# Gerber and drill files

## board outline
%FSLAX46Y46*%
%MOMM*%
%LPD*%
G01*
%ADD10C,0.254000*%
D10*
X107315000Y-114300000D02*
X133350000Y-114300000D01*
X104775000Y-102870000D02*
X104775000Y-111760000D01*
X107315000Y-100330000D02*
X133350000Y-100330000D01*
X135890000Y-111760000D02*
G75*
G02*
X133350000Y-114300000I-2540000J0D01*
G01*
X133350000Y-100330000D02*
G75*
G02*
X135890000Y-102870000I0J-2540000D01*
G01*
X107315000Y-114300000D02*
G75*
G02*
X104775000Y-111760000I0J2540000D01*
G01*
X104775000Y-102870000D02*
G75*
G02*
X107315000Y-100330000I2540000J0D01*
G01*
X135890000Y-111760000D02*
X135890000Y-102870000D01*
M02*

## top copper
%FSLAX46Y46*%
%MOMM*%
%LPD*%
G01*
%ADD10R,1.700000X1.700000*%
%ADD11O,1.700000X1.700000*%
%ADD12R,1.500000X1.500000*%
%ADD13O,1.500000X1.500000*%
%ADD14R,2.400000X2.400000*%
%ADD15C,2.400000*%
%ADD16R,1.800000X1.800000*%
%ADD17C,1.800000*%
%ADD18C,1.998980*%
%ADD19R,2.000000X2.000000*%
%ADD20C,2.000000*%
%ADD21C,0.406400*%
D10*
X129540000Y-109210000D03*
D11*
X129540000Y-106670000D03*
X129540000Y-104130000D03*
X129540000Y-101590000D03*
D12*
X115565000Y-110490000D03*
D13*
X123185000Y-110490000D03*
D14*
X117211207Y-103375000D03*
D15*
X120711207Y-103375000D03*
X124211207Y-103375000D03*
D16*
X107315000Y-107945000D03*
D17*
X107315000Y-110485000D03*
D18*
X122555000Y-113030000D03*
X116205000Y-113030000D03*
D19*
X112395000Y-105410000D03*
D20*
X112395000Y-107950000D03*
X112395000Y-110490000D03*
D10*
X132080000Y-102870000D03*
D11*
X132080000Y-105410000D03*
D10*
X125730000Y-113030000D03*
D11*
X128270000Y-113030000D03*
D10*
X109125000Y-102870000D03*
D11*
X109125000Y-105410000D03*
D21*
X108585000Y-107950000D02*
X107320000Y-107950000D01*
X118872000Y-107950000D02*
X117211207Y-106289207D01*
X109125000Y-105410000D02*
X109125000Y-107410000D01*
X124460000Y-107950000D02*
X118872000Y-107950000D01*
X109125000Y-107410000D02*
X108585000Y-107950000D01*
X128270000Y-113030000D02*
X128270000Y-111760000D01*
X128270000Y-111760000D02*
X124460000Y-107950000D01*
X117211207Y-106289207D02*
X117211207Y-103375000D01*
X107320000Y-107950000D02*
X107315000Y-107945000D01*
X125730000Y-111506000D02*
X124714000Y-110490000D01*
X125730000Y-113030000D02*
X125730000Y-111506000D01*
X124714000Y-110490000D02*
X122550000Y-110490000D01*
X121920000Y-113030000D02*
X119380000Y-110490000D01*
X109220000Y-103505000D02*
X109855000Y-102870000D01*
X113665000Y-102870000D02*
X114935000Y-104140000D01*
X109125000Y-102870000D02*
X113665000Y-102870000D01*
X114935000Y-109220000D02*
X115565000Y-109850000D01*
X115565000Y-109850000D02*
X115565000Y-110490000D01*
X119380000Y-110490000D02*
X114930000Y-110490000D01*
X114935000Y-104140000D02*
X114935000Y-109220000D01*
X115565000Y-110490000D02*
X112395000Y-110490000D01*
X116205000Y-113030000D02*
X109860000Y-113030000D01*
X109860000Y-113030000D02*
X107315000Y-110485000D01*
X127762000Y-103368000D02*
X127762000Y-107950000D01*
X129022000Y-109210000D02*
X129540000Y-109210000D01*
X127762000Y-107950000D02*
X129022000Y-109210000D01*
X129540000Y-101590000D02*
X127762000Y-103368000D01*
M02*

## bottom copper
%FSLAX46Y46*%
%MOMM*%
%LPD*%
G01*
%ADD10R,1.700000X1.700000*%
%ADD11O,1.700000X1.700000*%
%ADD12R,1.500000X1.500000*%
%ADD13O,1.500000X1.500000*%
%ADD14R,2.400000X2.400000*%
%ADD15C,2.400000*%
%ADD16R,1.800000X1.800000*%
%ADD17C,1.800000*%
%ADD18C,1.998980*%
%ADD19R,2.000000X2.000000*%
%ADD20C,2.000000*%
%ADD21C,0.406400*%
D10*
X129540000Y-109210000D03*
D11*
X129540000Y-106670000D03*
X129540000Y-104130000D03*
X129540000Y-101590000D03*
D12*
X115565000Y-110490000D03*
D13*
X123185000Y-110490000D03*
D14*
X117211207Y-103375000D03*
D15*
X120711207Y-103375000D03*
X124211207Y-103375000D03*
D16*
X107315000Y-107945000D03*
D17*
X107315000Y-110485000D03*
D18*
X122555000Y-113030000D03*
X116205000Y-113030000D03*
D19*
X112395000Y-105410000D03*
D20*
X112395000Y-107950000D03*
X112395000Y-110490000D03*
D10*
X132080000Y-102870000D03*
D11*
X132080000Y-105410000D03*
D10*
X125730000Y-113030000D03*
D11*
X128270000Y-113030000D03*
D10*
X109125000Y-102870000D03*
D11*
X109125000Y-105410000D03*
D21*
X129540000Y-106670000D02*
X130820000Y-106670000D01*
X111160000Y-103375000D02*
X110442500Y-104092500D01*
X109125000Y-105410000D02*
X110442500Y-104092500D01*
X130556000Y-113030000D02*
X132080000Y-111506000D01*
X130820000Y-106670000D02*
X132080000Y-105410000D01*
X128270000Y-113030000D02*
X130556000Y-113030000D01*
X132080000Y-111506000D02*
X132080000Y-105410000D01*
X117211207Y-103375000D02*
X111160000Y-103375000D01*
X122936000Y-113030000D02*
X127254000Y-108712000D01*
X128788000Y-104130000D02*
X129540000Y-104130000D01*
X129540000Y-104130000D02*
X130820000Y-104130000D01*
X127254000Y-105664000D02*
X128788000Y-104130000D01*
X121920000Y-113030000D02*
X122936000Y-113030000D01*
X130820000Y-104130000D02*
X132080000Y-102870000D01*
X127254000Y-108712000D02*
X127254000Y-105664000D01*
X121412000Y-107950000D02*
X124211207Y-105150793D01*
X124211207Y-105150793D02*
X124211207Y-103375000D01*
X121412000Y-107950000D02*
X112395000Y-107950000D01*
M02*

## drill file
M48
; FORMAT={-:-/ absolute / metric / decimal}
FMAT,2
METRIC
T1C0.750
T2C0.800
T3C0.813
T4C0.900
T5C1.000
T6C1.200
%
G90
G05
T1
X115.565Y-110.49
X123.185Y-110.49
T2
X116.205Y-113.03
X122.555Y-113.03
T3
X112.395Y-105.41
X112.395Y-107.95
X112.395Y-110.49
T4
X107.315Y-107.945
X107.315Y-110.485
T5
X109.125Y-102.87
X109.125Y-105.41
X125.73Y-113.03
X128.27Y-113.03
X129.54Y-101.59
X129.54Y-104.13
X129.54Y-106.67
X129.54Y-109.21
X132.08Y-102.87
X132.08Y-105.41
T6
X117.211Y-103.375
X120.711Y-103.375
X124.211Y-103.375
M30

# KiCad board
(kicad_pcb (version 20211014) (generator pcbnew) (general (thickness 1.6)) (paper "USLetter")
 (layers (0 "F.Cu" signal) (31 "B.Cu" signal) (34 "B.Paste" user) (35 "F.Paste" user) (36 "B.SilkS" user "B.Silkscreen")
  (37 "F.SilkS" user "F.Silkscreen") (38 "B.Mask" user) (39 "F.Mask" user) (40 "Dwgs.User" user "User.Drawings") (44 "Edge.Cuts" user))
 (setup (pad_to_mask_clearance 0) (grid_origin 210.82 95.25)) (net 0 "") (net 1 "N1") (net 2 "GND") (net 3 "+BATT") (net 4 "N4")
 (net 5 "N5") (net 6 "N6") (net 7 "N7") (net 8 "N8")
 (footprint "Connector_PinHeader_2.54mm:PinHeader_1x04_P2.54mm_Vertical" (layer "F.Cu") (at 129.54 109.21 180)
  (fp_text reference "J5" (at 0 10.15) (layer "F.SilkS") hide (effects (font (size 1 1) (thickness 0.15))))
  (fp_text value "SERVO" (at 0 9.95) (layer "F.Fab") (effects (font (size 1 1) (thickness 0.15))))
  (pad "1" thru_hole rect (at 0 0 180) (size 1.7 1.7) (drill 1) (layers *.Cu *.Mask) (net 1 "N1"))
  (pad "2" thru_hole oval (at 0 2.54 180) (size 1.7 1.7) (drill 1) (layers *.Cu *.Mask) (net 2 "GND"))
  (pad "3" thru_hole oval (at 0 5.08 180) (size 1.7 1.7) (drill 1) (layers *.Cu *.Mask) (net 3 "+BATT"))
  (pad "4" thru_hole oval (at 0 7.62 180) (size 1.7 1.7) (drill 1) (layers *.Cu *.Mask) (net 1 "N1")))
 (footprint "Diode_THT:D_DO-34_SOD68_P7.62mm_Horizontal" (layer "F.Cu") (at 115.565 110.49)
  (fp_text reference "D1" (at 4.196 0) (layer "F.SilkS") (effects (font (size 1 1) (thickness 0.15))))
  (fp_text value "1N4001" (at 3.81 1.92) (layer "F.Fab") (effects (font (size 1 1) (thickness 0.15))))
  (pad "1" thru_hole rect (at 0 0) (size 1.5 1.5) (drill 0.75) (layers *.Cu *.Mask) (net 3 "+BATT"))
  (pad "2" thru_hole oval (at 7.62 0) (size 1.5 1.5) (drill 0.75) (layers *.Cu *.Mask) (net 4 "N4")))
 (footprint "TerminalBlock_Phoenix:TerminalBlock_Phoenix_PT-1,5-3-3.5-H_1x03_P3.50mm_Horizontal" (layer "F.Cu") (at 117.211207 103.375)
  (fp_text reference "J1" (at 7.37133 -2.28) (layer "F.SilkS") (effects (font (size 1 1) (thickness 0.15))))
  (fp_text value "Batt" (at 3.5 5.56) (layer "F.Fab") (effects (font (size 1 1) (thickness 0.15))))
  (pad "1" thru_hole rect (at 0 0) (size 2.4 2.4) (drill 1.2) (layers *.Cu *.Mask) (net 2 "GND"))
  (pad "2" thru_hole circle (at 3.5 0) (size 2.4 2.4) (drill 1.2) (layers *.Cu *.Mask) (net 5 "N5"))
  (pad "3" thru_hole circle (at 7 0) (size 2.4 2.4) (drill 1.2) (layers *.Cu *.Mask) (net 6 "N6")))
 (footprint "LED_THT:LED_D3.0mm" (layer "F.Cu") (at 107.315 107.945 -90)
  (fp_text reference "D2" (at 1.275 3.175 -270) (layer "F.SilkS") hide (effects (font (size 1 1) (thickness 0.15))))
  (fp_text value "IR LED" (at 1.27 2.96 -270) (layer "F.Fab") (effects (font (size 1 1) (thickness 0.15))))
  (pad "1" thru_hole rect (at 0 0 270) (size 1.8 1.8) (drill 0.9) (layers *.Cu *.Mask) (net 2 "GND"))
  (pad "2" thru_hole circle (at 2.54 0 270) (size 1.8 1.8) (drill 0.9) (layers *.Cu *.Mask) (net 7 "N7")))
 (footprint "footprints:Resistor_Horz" (layer "F.Cu") (at 119.38 113.03 180)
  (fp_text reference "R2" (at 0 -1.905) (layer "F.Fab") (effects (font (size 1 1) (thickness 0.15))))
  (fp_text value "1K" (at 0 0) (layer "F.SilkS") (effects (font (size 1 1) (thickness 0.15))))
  (pad "1" thru_hole circle (at -3.175 0 180) (size 1.99898 1.99898) (drill 0.8) (layers *.Cu *.SilkS *.Mask) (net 3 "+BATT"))
  (pad "2" thru_hole circle (at 3.175 0 180) (size 1.99898 1.99898) (drill 0.8) (layers *.Cu *.SilkS *.Mask) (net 7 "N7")))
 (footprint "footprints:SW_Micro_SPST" (layer "F.Cu") (at 112.395 107.95 -90)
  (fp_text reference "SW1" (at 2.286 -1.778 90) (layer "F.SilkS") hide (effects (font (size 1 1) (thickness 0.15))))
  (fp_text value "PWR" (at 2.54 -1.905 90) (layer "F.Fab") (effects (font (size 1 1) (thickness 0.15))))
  (pad "1" thru_hole rect (at -2.54 0 270) (size 2 2) (drill 0.8128) (layers *.Cu *.Mask "F.SilkS") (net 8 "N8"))
  (pad "2" thru_hole circle (at 0 0 270) (size 2 2) (drill 0.8128) (layers *.Cu *.Mask "F.SilkS") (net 6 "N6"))
  (pad "3" thru_hole circle (at 2.54 0 270) (size 2 2) (drill 0.8128) (layers *.Cu *.Mask "F.SilkS") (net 3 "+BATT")))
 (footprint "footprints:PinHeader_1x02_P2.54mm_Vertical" (layer "B.Cu") (at 132.08 102.87 180)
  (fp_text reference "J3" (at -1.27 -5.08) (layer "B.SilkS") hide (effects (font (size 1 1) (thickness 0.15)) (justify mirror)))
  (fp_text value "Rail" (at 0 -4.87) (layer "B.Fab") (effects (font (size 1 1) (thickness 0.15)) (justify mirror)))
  (pad "1" thru_hole rect (at 0 0 180) (size 1.7 1.7) (drill 1) (layers *.Cu *.Mask) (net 3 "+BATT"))
  (pad "2" thru_hole oval (at 0 -2.54 180) (size 1.7 1.7) (drill 1) (layers *.Cu *.Mask) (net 2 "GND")))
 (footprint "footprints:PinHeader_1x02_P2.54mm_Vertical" (layer "B.Cu") (at 125.73 113.03 -90)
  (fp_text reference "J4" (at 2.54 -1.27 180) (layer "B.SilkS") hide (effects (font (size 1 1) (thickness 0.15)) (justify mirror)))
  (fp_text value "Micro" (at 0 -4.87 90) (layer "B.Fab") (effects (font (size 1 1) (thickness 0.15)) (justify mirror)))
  (pad "1" thru_hole rect (at 0 0 270) (size 1.7 1.7) (drill 1) (layers *.Cu *.Mask) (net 4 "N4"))
  (pad "2" thru_hole oval (at 0 -2.54 270) (size 1.7 1.7) (drill 1) (layers *.Cu *.Mask) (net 2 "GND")))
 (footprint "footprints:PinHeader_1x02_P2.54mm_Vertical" (layer "B.Cu") (at 109.125 102.87 180)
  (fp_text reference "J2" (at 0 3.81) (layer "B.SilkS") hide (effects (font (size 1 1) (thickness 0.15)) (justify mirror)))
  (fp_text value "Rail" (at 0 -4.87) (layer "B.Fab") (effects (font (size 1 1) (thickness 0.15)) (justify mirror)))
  (pad "1" thru_hole rect (at 0 0 180) (size 1.7 1.7) (drill 1) (layers *.Cu *.Mask) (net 3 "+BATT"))
  (pad "2" thru_hole oval (at 0 -2.54 180) (size 1.7 1.7) (drill 1) (layers *.Cu *.Mask) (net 2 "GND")))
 (gr_line (start 107.315 114.3) (end 133.35 114.3) (layer "Edge.Cuts") (width 0.254))
 (gr_line (start 104.775 102.87) (end 104.775 111.76) (layer "Edge.Cuts") (width 0.254))
 (gr_line (start 107.315 100.33) (end 133.35 100.33) (layer "Edge.Cuts") (width 0.254))
 (gr_arc (start 135.89 111.76) (mid 135.146051 113.556051) (end 133.35 114.3) (layer "Edge.Cuts") (width 0.254))
 (gr_arc (start 133.35 100.33) (mid 135.146051 101.073949) (end 135.89 102.87) (layer "Edge.Cuts") (width 0.254))
 (gr_arc (start 107.315 114.3) (mid 105.518949 113.556051) (end 104.775 111.76) (layer "Edge.Cuts") (width 0.254))
 (gr_arc (start 104.775 102.87) (mid 105.518949 101.073949) (end 107.315 100.33) (layer "Edge.Cuts") (width 0.254))
 (gr_line (start 135.89 111.76) (end 135.89 102.87) (layer "Edge.Cuts") (width 0.254))
 (segment (start 108.585 107.95) (end 107.32 107.95) (width 0.4064) (layer "F.Cu") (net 2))
 (segment (start 118.872 107.95) (end 117.211207 106.289207) (width 0.4064) (layer "F.Cu") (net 2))
 (segment (start 109.125 105.41) (end 109.125 107.41) (width 0.4064) (layer "F.Cu") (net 2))
 (segment (start 124.46 107.95) (end 118.872 107.95) (width 0.4064) (layer "F.Cu") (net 2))
 (segment (start 109.125 107.41) (end 108.585 107.95) (width 0.4064) (layer "F.Cu") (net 2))
 (segment (start 128.27 113.03) (end 128.27 111.76) (width 0.4064) (layer "F.Cu") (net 2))
 (segment (start 128.27 111.76) (end 124.46 107.95) (width 0.4064) (layer "F.Cu") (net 2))
 (segment (start 117.211207 106.289207) (end 117.211207 103.375) (width 0.4064) (layer "F.Cu") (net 2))
 (segment (start 107.32 107.95) (end 107.315 107.945) (width 0.4064) (layer "F.Cu") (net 2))
 (segment (start 129.54 106.67) (end 130.82 106.67) (width 0.4064) (layer "B.Cu") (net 2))
 (segment (start 111.16 103.375) (end 110.4425 104.0925) (width 0.4064) (layer "B.Cu") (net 2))
 (segment (start 109.125 105.41) (end 110.4425 104.0925) (width 0.4064) (layer "B.Cu") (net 2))
 (segment (start 130.556 113.03) (end 132.08 111.506) (width 0.4064) (layer "B.Cu") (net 2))
 (segment (start 130.82 106.67) (end 132.08 105.41) (width 0.4064) (layer "B.Cu") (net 2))
 (segment (start 128.27 113.03) (end 130.556 113.03) (width 0.4064) (layer "B.Cu") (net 2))
 (segment (start 132.08 111.506) (end 132.08 105.41) (width 0.4064) (layer "B.Cu") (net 2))
 (segment (start 117.211207 103.375) (end 111.16 103.375) (width 0.4064) (layer "B.Cu") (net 2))
 (segment (start 125.73 111.506) (end 124.714 110.49) (width 0.4064) (layer "F.Cu") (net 4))
 (segment (start 125.73 113.03) (end 125.73 111.506) (width 0.4064) (layer "F.Cu") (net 4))
 (segment (start 124.714 110.49) (end 122.55 110.49) (width 0.4064) (layer "F.Cu") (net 4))
 (segment (start 121.92 113.03) (end 119.38 110.49) (width 0.4064) (layer "F.Cu") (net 3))
 (segment (start 109.22 103.505) (end 109.855 102.87) (width 0.4064) (layer "F.Cu") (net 3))
 (segment (start 113.665 102.87) (end 114.935 104.14) (width 0.4064) (layer "F.Cu") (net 3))
 (segment (start 109.125 102.87) (end 113.665 102.87) (width 0.4064) (layer "F.Cu") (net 3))
 (segment (start 114.935 109.22) (end 115.565 109.85) (width 0.4064) (layer "F.Cu") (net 3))
 (segment (start 115.565 109.85) (end 115.565 110.49) (width 0.4064) (layer "F.Cu") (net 3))
 (segment (start 119.38 110.49) (end 114.93 110.49) (width 0.4064) (layer "F.Cu") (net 3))
 (segment (start 114.935 104.14) (end 114.935 109.22) (width 0.4064) (layer "F.Cu") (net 3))
 (segment (start 115.565 110.49) (end 112.395 110.49) (width 0.4064) (layer "F.Cu") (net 3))
 (segment (start 122.936 113.03) (end 127.254 108.712) (width 0.4064) (layer "B.Cu") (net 3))
 (segment (start 128.788 104.13) (end 129.54 104.13) (width 0.4064) (layer "B.Cu") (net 3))
 (segment (start 129.54 104.13) (end 130.82 104.13) (width 0.4064) (layer "B.Cu") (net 3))
 (segment (start 127.254 105.664) (end 128.788 104.13) (width 0.4064) (layer "B.Cu") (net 3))
 (segment (start 121.92 113.03) (end 122.936 113.03) (width 0.4064) (layer "B.Cu") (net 3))
 (segment (start 130.82 104.13) (end 132.08 102.87) (width 0.4064) (layer "B.Cu") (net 3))
 (segment (start 127.254 108.712) (end 127.254 105.664) (width 0.4064) (layer "B.Cu") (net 3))
 (segment (start 116.205 113.03) (end 109.86 113.03) (width 0.4064) (layer "F.Cu") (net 7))
 (segment (start 109.86 113.03) (end 107.315 110.485) (width 0.4064) (layer "F.Cu") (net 7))
 (segment (start 121.412 107.95) (end 124.211207 105.150793) (width 0.4064) (layer "B.Cu") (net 6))
 (segment (start 124.211207 105.150793) (end 124.211207 103.375) (width 0.4064) (layer "B.Cu") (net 6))
 (segment (start 121.412 107.95) (end 112.395 107.95) (width 0.4064) (layer "B.Cu") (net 6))
 (segment (start 127.762 103.368) (end 127.762 107.95) (width 0.4064) (layer "F.Cu") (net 1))
 (segment (start 129.022 109.21) (end 129.54 109.21) (width 0.4064) (layer "F.Cu") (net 1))
 (segment (start 127.762 107.95) (end 129.022 109.21) (width 0.4064) (layer "F.Cu") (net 1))
 (segment (start 129.54 101.59) (end 127.762 103.368) (width 0.4064) (layer "F.Cu") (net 1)))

